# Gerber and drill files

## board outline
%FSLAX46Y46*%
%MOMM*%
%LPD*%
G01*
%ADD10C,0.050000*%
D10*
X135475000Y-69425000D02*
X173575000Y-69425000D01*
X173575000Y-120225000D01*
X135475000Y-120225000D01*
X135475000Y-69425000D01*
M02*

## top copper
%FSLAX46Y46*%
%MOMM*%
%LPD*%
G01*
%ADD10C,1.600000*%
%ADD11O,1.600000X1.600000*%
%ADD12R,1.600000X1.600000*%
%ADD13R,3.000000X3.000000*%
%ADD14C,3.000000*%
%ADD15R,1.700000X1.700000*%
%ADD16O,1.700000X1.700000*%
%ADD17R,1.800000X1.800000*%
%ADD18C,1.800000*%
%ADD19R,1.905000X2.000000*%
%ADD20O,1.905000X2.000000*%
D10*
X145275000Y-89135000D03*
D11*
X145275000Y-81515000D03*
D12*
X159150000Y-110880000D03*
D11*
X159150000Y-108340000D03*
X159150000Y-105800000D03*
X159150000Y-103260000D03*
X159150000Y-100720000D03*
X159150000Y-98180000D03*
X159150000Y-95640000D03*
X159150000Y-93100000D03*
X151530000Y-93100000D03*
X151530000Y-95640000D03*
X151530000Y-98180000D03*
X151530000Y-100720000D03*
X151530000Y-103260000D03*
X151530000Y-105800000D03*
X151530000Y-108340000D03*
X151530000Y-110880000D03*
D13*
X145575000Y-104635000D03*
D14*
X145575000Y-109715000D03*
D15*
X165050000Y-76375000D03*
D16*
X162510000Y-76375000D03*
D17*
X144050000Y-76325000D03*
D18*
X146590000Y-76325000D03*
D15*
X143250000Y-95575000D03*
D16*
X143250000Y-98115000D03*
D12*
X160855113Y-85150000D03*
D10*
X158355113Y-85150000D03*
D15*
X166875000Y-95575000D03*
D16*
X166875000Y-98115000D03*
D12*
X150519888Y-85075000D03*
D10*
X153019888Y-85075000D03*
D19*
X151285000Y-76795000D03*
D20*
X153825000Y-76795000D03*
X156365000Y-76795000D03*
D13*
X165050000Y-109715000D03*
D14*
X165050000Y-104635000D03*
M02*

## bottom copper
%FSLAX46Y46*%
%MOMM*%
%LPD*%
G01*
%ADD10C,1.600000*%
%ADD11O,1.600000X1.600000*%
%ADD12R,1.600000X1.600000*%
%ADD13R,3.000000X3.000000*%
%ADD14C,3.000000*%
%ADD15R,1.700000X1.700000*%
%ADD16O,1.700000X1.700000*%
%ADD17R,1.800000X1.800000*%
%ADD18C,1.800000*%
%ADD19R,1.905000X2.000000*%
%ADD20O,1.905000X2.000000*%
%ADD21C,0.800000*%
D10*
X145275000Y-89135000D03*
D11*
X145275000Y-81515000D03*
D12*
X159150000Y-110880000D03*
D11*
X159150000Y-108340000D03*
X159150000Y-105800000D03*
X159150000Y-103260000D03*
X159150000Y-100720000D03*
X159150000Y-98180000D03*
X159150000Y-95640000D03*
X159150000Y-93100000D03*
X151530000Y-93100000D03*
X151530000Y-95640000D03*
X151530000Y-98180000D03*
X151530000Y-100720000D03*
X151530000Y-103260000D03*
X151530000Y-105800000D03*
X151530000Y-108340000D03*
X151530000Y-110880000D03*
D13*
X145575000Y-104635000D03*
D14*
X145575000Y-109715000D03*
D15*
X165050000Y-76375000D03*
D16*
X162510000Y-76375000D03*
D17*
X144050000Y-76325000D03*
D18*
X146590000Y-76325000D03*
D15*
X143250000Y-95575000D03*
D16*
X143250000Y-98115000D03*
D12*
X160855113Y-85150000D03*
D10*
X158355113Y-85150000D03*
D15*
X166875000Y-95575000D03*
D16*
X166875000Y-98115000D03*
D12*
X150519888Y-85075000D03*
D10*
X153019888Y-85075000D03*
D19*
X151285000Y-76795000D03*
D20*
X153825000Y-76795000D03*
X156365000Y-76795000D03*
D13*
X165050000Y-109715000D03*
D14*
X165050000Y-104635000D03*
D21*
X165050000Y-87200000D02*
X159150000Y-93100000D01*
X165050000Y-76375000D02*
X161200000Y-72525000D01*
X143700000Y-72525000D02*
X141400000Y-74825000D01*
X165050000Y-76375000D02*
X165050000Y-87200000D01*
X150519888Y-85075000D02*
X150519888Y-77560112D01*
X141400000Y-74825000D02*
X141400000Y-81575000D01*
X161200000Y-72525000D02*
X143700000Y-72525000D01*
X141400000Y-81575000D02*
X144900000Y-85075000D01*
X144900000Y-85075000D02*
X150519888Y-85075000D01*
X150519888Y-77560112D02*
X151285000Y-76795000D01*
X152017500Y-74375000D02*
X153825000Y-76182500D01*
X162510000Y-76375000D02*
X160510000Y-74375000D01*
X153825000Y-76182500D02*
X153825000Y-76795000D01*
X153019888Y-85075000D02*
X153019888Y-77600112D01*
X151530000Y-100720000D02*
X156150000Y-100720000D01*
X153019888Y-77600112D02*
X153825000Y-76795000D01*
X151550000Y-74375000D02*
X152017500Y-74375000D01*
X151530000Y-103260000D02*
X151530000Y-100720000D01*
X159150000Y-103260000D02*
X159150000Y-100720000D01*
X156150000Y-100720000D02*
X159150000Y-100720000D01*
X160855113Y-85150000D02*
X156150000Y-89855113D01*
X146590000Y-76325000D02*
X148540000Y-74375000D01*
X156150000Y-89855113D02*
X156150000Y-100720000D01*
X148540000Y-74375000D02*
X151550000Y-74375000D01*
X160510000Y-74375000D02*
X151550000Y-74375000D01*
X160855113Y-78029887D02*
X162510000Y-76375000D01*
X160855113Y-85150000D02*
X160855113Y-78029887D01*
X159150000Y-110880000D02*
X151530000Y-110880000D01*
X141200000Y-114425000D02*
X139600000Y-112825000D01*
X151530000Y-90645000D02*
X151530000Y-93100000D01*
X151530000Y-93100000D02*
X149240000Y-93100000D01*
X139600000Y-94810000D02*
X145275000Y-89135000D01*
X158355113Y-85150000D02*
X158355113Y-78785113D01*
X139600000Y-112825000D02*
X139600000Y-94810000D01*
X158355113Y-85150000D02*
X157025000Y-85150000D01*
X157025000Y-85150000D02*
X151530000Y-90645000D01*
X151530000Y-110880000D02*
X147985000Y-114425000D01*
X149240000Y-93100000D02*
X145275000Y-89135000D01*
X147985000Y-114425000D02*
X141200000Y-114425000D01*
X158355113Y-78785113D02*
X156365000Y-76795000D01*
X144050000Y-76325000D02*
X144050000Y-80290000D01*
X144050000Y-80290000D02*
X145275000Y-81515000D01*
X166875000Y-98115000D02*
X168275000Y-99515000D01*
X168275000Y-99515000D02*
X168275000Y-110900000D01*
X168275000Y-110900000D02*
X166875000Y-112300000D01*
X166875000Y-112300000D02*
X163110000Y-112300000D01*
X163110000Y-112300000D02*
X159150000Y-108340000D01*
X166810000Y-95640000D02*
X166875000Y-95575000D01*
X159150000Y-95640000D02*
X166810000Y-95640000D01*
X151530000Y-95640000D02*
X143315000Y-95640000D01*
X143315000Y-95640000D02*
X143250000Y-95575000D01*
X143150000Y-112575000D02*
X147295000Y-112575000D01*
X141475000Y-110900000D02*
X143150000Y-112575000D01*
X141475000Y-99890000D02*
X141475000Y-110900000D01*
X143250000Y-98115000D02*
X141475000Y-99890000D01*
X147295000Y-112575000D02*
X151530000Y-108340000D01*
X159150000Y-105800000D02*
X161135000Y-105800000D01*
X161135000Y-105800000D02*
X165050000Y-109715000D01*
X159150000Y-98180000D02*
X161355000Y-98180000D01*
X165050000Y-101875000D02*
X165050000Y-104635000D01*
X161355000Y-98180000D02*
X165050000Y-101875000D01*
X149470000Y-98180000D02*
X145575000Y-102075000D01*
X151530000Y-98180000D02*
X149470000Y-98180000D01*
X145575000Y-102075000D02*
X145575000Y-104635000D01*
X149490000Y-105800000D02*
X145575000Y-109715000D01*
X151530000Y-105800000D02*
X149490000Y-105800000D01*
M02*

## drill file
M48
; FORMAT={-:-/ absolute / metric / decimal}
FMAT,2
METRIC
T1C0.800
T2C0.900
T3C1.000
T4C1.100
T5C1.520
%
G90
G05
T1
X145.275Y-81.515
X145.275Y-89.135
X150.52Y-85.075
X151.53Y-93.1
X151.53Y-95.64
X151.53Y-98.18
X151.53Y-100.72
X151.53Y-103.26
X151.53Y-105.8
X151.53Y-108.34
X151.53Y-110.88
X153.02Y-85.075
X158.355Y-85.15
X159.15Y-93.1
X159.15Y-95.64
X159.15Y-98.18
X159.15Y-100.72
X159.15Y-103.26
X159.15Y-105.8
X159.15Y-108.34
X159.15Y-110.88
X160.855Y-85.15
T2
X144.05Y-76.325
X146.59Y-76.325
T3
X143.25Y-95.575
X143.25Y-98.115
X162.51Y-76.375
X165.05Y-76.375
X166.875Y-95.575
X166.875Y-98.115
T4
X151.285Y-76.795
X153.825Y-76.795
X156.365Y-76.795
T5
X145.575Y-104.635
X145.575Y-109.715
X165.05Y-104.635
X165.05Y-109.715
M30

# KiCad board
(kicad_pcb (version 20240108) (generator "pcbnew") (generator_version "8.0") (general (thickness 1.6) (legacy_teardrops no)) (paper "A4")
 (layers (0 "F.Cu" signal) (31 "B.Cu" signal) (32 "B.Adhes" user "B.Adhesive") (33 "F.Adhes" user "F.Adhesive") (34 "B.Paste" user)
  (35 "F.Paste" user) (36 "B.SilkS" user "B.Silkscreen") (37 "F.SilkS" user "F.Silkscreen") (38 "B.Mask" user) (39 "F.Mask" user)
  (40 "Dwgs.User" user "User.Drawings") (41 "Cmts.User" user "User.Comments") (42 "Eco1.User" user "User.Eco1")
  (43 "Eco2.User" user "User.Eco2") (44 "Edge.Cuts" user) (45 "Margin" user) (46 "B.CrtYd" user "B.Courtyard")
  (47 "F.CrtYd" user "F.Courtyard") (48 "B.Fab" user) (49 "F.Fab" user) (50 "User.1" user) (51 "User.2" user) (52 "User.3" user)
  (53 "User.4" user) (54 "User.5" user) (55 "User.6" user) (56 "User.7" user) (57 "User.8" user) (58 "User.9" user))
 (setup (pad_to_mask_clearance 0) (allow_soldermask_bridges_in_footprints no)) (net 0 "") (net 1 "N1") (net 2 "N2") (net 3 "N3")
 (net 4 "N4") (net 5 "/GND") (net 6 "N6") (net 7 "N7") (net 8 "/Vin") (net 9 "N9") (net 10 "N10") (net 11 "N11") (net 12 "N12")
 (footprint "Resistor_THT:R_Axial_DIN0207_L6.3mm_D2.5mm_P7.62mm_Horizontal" (layer "F.Cu") (at 145.275 89.135 90)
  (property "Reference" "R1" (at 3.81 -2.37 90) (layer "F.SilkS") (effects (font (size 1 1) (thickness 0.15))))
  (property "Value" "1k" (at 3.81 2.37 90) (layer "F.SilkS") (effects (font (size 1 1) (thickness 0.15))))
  (pad "1" thru_hole circle (at 0 0 90) (size 1.6 1.6) (drill 0.8) (layers "*.Cu" "*.Mask") (remove_unused_layers no) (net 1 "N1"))
  (pad "2" thru_hole oval (at 7.62 0 90) (size 1.6 1.6) (drill 0.8) (layers "*.Cu" "*.Mask") (remove_unused_layers no) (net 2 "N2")))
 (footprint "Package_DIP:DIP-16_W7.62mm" (layer "F.Cu") (at 159.15 110.88 180)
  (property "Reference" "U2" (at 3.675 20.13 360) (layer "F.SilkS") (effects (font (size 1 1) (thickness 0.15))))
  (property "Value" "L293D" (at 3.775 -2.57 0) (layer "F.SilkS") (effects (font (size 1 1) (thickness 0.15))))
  (pad "1" thru_hole rect (at 0 0 180) (size 1.6 1.6) (drill 0.8) (layers "*.Cu" "*.Mask") (remove_unused_layers no) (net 1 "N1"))
  (pad "2" thru_hole oval (at 0 2.54 180) (size 1.6 1.6) (drill 0.8) (layers "*.Cu" "*.Mask") (remove_unused_layers no) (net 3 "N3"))
  (pad "3" thru_hole oval (at 0 5.08 180) (size 1.6 1.6) (drill 0.8) (layers "*.Cu" "*.Mask") (remove_unused_layers no) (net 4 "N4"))
  (pad "4" thru_hole oval (at 0 7.62 180) (size 1.6 1.6) (drill 0.8) (layers "*.Cu" "*.Mask") (remove_unused_layers no) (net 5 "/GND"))
  (pad "5" thru_hole oval (at 0 10.16 180) (size 1.6 1.6) (drill 0.8) (layers "*.Cu" "*.Mask") (remove_unused_layers no) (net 5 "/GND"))
  (pad "6" thru_hole oval (at 0 12.7 180) (size 1.6 1.6) (drill 0.8) (layers "*.Cu" "*.Mask") (remove_unused_layers no) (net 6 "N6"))
  (pad "7" thru_hole oval (at 0 15.24 180) (size 1.6 1.6) (drill 0.8) (layers "*.Cu" "*.Mask") (remove_unused_layers no) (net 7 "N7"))
  (pad "8" thru_hole oval (at 0 17.78 180) (size 1.6 1.6) (drill 0.8) (layers "*.Cu" "*.Mask") (remove_unused_layers no) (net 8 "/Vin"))
  (pad "9" thru_hole oval (at 7.62 17.78 180) (size 1.6 1.6) (drill 0.8) (layers "*.Cu" "*.Mask") (remove_unused_layers no) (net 1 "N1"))
  (pad "10" thru_hole oval (at 7.62 15.24 180) (size 1.6 1.6) (drill 0.8) (layers "*.Cu" "*.Mask") (remove_unused_layers no) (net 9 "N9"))
  (pad "11" thru_hole oval (at 7.62 12.7 180) (size 1.6 1.6) (drill 0.8) (layers "*.Cu" "*.Mask") (remove_unused_layers no) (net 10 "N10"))
  (pad "12" thru_hole oval (at 7.62 10.16 180) (size 1.6 1.6) (drill 0.8) (layers "*.Cu" "*.Mask") (remove_unused_layers no) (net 5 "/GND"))
  (pad "13" thru_hole oval (at 7.62 7.62 180) (size 1.6 1.6) (drill 0.8) (layers "*.Cu" "*.Mask") (remove_unused_layers no) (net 5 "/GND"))
  (pad "14" thru_hole oval (at 7.62 5.08 180) (size 1.6 1.6) (drill 0.8) (layers "*.Cu" "*.Mask") (remove_unused_layers no) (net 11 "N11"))
  (pad "15" thru_hole oval (at 7.62 2.54 180) (size 1.6 1.6) (drill 0.8) (layers "*.Cu" "*.Mask") (remove_unused_layers no) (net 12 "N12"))
  (pad "16" thru_hole oval (at 7.62 0 180) (size 1.6 1.6) (drill 0.8) (layers "*.Cu" "*.Mask") (remove_unused_layers no) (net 1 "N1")))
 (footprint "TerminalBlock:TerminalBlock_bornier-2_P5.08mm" (layer "F.Cu") (at 145.575 104.635 -90)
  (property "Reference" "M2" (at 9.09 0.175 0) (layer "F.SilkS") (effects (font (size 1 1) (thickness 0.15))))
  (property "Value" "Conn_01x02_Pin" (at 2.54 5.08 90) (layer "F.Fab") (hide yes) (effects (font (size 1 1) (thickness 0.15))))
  (pad "1" thru_hole rect (at 0 0 270) (size 3 3) (drill 1.52) (layers "*.Cu" "*.Mask") (remove_unused_layers no) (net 10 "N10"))
  (pad "2" thru_hole circle (at 5.08 0 270) (size 3 3) (drill 1.52) (layers "*.Cu" "*.Mask") (remove_unused_layers no) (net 11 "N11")))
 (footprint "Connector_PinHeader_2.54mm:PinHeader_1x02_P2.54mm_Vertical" (layer "F.Cu") (at 165.05 76.375 -90)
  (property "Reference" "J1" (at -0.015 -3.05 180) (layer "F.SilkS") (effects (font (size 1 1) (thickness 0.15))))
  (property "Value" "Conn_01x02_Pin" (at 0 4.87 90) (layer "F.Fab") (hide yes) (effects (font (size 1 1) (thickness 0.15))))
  (pad "1" thru_hole rect (at 0 0 270) (size 1.7 1.7) (drill 1) (layers "*.Cu" "*.Mask") (remove_unused_layers no) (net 8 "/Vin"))
  (pad "2" thru_hole oval (at 0 2.54 270) (size 1.7 1.7) (drill 1) (layers "*.Cu" "*.Mask") (remove_unused_layers no) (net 5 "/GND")))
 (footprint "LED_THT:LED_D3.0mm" (layer "F.Cu") (at 144.05 76.325)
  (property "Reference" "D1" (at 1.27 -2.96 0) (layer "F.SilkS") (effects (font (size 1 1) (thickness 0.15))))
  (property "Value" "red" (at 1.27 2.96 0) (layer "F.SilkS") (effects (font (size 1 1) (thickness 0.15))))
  (pad "1" thru_hole rect (at 0 0) (size 1.8 1.8) (drill 0.9) (layers "*.Cu" "*.Mask") (remove_unused_layers no) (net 2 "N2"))
  (pad "2" thru_hole circle (at 2.54 0) (size 1.8 1.8) (drill 0.9) (layers "*.Cu" "*.Mask") (remove_unused_layers no) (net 5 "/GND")))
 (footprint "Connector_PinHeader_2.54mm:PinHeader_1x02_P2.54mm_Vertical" (layer "F.Cu") (at 143.25 95.575)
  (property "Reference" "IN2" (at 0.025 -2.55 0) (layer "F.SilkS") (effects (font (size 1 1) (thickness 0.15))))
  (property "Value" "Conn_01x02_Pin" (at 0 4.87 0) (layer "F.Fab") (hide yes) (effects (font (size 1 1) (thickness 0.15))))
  (pad "1" thru_hole rect (at 0 0) (size 1.7 1.7) (drill 1) (layers "*.Cu" "*.Mask") (remove_unused_layers no) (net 9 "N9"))
  (pad "2" thru_hole oval (at 0 2.54) (size 1.7 1.7) (drill 1) (layers "*.Cu" "*.Mask") (remove_unused_layers no) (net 12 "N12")))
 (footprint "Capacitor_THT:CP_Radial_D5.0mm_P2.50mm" (layer "F.Cu") (at 160.855113 85.15 180)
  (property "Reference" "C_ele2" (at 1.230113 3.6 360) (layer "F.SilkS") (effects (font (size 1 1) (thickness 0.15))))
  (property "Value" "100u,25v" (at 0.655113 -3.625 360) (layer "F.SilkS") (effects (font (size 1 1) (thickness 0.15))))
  (pad "1" thru_hole rect (at 0 0 180) (size 1.6 1.6) (drill 0.8) (layers "*.Cu" "*.Mask") (remove_unused_layers no) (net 5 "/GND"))
  (pad "2" thru_hole circle (at 2.5 0 180) (size 1.6 1.6) (drill 0.8) (layers "*.Cu" "*.Mask") (remove_unused_layers no) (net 1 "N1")))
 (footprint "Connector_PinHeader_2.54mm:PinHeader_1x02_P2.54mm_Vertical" (layer "F.Cu") (at 166.875 95.575)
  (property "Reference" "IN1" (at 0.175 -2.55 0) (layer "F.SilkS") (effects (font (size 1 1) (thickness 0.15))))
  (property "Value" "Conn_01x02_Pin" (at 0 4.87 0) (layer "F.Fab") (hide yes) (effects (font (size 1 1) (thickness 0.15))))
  (pad "1" thru_hole rect (at 0 0) (size 1.7 1.7) (drill 1) (layers "*.Cu" "*.Mask") (remove_unused_layers no) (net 7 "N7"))
  (pad "2" thru_hole oval (at 0 2.54) (size 1.7 1.7) (drill 1) (layers "*.Cu" "*.Mask") (remove_unused_layers no) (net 3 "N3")))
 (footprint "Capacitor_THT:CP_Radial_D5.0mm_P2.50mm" (layer "F.Cu") (at 150.519888 85.075)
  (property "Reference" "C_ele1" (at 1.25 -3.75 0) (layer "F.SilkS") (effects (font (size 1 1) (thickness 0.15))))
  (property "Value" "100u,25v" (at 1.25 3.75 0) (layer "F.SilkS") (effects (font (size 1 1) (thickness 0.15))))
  (pad "1" thru_hole rect (at 0 0) (size 1.6 1.6) (drill 0.8) (layers "*.Cu" "*.Mask") (remove_unused_layers no) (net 8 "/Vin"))
  (pad "2" thru_hole circle (at 2.5 0) (size 1.6 1.6) (drill 0.8) (layers "*.Cu" "*.Mask") (remove_unused_layers no) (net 5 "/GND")))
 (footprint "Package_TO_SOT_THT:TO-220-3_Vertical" (layer "F.Cu") (at 151.285 76.795)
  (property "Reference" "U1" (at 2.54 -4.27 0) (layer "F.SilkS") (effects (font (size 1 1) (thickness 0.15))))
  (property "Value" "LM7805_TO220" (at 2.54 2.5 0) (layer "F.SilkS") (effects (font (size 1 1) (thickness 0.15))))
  (pad "1" thru_hole rect (at 0 0) (size 1.905 2) (drill 1.1) (layers "*.Cu" "*.Mask") (remove_unused_layers no) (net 8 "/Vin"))
  (pad "2" thru_hole oval (at 2.54 0) (size 1.905 2) (drill 1.1) (layers "*.Cu" "*.Mask") (remove_unused_layers no) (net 5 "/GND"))
  (pad "3" thru_hole oval (at 5.08 0) (size 1.905 2) (drill 1.1) (layers "*.Cu" "*.Mask") (remove_unused_layers no) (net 1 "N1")))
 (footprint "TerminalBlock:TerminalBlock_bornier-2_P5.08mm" (layer "F.Cu") (at 165.05 109.715 90)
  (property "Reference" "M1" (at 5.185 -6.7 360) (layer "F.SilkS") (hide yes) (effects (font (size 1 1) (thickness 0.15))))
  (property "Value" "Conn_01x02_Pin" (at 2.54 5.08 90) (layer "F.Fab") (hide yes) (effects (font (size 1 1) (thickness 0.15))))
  (pad "1" thru_hole rect (at 0 0 90) (size 3 3) (drill 1.52) (layers "*.Cu" "*.Mask") (remove_unused_layers no) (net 4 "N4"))
  (pad "2" thru_hole circle (at 5.08 0 90) (size 3 3) (drill 1.52) (layers "*.Cu" "*.Mask") (remove_unused_layers no) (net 6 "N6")))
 (gr_rect (start 135.475 69.425) (end 173.575 120.225) (stroke (width 0.05) (type default)) (fill none) (layer "Edge.Cuts"))
 (segment (start 165.05 87.2) (end 159.15 93.1) (width 0.8) (layer "B.Cu") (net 8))
 (segment (start 165.05 76.375) (end 161.2 72.525) (width 0.8) (layer "B.Cu") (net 8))
 (segment (start 143.7 72.525) (end 141.4 74.825) (width 0.8) (layer "B.Cu") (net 8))
 (segment (start 165.05 76.375) (end 165.05 87.2) (width 0.8) (layer "B.Cu") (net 8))
 (segment (start 150.519888 85.075) (end 150.519888 77.560112) (width 0.8) (layer "B.Cu") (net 8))
 (segment (start 141.4 74.825) (end 141.4 81.575) (width 0.8) (layer "B.Cu") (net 8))
 (segment (start 161.2 72.525) (end 143.7 72.525) (width 0.8) (layer "B.Cu") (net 8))
 (segment (start 141.4 81.575) (end 144.9 85.075) (width 0.8) (layer "B.Cu") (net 8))
 (segment (start 144.9 85.075) (end 150.519888 85.075) (width 0.8) (layer "B.Cu") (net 8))
 (segment (start 150.519888 77.560112) (end 151.285 76.795) (width 0.8) (layer "B.Cu") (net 8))
 (segment (start 152.0175 74.375) (end 153.825 76.1825) (width 0.8) (layer "B.Cu") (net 5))
 (segment (start 162.51 76.375) (end 160.51 74.375) (width 0.8) (layer "B.Cu") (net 5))
 (segment (start 153.825 76.1825) (end 153.825 76.795) (width 0.8) (layer "B.Cu") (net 5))
 (segment (start 153.019888 85.075) (end 153.019888 77.600112) (width 0.8) (layer "B.Cu") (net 5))
 (segment (start 151.53 100.72) (end 156.15 100.72) (width 0.8) (layer "B.Cu") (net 5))
 (segment (start 153.019888 77.600112) (end 153.825 76.795) (width 0.8) (layer "B.Cu") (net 5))
 (segment (start 151.55 74.375) (end 152.0175 74.375) (width 0.8) (layer "B.Cu") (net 5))
 (segment (start 151.53 103.26) (end 151.53 100.72) (width 0.8) (layer "B.Cu") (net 5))
 (segment (start 159.15 103.26) (end 159.15 100.72) (width 0.8) (layer "B.Cu") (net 5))
 (segment (start 156.15 100.72) (end 159.15 100.72) (width 0.8) (layer "B.Cu") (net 5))
 (segment (start 160.855113 85.15) (end 156.15 89.855113) (width 0.8) (layer "B.Cu") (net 5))
 (segment (start 146.59 76.325) (end 148.54 74.375) (width 0.8) (layer "B.Cu") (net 5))
 (segment (start 156.15 89.855113) (end 156.15 100.72) (width 0.8) (layer "B.Cu") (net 5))
 (segment (start 148.54 74.375) (end 151.55 74.375) (width 0.8) (layer "B.Cu") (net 5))
 (segment (start 160.51 74.375) (end 151.55 74.375) (width 0.8) (layer "B.Cu") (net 5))
 (segment (start 160.855113 78.029887) (end 162.51 76.375) (width 0.8) (layer "B.Cu") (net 5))
 (segment (start 160.855113 85.15) (end 160.855113 78.029887) (width 0.8) (layer "B.Cu") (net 5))
 (segment (start 159.15 110.88) (end 151.53 110.88) (width 0.8) (layer "B.Cu") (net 1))
 (segment (start 141.2 114.425) (end 139.6 112.825) (width 0.8) (layer "B.Cu") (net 1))
 (segment (start 151.53 90.645) (end 151.53 93.1) (width 0.8) (layer "B.Cu") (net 1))
 (segment (start 151.53 93.1) (end 149.24 93.1) (width 0.8) (layer "B.Cu") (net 1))
 (segment (start 139.6 94.81) (end 145.275 89.135) (width 0.8) (layer "B.Cu") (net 1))
 (segment (start 158.355113 85.15) (end 158.355113 78.785113) (width 0.8) (layer "B.Cu") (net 1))
 (segment (start 139.6 112.825) (end 139.6 94.81) (width 0.8) (layer "B.Cu") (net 1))
 (segment (start 158.355113 85.15) (end 157.025 85.15) (width 0.8) (layer "B.Cu") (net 1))
 (segment (start 157.025 85.15) (end 151.53 90.645) (width 0.8) (layer "B.Cu") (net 1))
 (segment (start 151.53 110.88) (end 147.985 114.425) (width 0.8) (layer "B.Cu") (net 1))
 (segment (start 149.24 93.1) (end 145.275 89.135) (width 0.8) (layer "B.Cu") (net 1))
 (segment (start 147.985 114.425) (end 141.2 114.425) (width 0.8) (layer "B.Cu") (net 1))
 (segment (start 158.355113 78.785113) (end 156.365 76.795) (width 0.8) (layer "B.Cu") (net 1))
 (segment (start 144.05 76.325) (end 144.05 80.29) (width 0.8) (layer "B.Cu") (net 2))
 (segment (start 144.05 80.29) (end 145.275 81.515) (width 0.8) (layer "B.Cu") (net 2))
 (segment (start 166.875 98.115) (end 168.275 99.515) (width 0.8) (layer "B.Cu") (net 3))
 (segment (start 168.275 99.515) (end 168.275 110.9) (width 0.8) (layer "B.Cu") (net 3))
 (segment (start 168.275 110.9) (end 166.875 112.3) (width 0.8) (layer "B.Cu") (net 3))
 (segment (start 166.875 112.3) (end 163.11 112.3) (width 0.8) (layer "B.Cu") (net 3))
 (segment (start 163.11 112.3) (end 159.15 108.34) (width 0.8) (layer "B.Cu") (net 3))
 (segment (start 166.81 95.64) (end 166.875 95.575) (width 0.8) (layer "B.Cu") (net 7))
 (segment (start 159.15 95.64) (end 166.81 95.64) (width 0.8) (layer "B.Cu") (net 7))
 (segment (start 151.53 95.64) (end 143.315 95.64) (width 0.8) (layer "B.Cu") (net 9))
 (segment (start 143.315 95.64) (end 143.25 95.575) (width 0.8) (layer "B.Cu") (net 9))
 (segment (start 143.15 112.575) (end 147.295 112.575) (width 0.8) (layer "B.Cu") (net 12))
 (segment (start 141.475 110.9) (end 143.15 112.575) (width 0.8) (layer "B.Cu") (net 12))
 (segment (start 141.475 99.89) (end 141.475 110.9) (width 0.8) (layer "B.Cu") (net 12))
 (segment (start 143.25 98.115) (end 141.475 99.89) (width 0.8) (layer "B.Cu") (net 12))
 (segment (start 147.295 112.575) (end 151.53 108.34) (width 0.8) (layer "B.Cu") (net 12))
 (segment (start 159.15 105.8) (end 161.135 105.8) (width 0.8) (layer "B.Cu") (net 4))
 (segment (start 161.135 105.8) (end 165.05 109.715) (width 0.8) (layer "B.Cu") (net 4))
 (segment (start 159.15 98.18) (end 161.355 98.18) (width 0.8) (layer "B.Cu") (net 6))
 (segment (start 165.05 101.875) (end 165.05 104.635) (width 0.8) (layer "B.Cu") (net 6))
 (segment (start 161.355 98.18) (end 165.05 101.875) (width 0.8) (layer "B.Cu") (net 6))
 (segment (start 149.47 98.18) (end 145.575 102.075) (width 0.8) (layer "B.Cu") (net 10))
 (segment (start 151.53 98.18) (end 149.47 98.18) (width 0.8) (layer "B.Cu") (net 10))
 (segment (start 145.575 102.075) (end 145.575 104.635) (width 0.8) (layer "B.Cu") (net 10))
 (segment (start 149.49 105.8) (end 145.575 109.715) (width 0.8) (layer "B.Cu") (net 11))
 (segment (start 151.53 105.8) (end 149.49 105.8) (width 0.8) (layer "B.Cu") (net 11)))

